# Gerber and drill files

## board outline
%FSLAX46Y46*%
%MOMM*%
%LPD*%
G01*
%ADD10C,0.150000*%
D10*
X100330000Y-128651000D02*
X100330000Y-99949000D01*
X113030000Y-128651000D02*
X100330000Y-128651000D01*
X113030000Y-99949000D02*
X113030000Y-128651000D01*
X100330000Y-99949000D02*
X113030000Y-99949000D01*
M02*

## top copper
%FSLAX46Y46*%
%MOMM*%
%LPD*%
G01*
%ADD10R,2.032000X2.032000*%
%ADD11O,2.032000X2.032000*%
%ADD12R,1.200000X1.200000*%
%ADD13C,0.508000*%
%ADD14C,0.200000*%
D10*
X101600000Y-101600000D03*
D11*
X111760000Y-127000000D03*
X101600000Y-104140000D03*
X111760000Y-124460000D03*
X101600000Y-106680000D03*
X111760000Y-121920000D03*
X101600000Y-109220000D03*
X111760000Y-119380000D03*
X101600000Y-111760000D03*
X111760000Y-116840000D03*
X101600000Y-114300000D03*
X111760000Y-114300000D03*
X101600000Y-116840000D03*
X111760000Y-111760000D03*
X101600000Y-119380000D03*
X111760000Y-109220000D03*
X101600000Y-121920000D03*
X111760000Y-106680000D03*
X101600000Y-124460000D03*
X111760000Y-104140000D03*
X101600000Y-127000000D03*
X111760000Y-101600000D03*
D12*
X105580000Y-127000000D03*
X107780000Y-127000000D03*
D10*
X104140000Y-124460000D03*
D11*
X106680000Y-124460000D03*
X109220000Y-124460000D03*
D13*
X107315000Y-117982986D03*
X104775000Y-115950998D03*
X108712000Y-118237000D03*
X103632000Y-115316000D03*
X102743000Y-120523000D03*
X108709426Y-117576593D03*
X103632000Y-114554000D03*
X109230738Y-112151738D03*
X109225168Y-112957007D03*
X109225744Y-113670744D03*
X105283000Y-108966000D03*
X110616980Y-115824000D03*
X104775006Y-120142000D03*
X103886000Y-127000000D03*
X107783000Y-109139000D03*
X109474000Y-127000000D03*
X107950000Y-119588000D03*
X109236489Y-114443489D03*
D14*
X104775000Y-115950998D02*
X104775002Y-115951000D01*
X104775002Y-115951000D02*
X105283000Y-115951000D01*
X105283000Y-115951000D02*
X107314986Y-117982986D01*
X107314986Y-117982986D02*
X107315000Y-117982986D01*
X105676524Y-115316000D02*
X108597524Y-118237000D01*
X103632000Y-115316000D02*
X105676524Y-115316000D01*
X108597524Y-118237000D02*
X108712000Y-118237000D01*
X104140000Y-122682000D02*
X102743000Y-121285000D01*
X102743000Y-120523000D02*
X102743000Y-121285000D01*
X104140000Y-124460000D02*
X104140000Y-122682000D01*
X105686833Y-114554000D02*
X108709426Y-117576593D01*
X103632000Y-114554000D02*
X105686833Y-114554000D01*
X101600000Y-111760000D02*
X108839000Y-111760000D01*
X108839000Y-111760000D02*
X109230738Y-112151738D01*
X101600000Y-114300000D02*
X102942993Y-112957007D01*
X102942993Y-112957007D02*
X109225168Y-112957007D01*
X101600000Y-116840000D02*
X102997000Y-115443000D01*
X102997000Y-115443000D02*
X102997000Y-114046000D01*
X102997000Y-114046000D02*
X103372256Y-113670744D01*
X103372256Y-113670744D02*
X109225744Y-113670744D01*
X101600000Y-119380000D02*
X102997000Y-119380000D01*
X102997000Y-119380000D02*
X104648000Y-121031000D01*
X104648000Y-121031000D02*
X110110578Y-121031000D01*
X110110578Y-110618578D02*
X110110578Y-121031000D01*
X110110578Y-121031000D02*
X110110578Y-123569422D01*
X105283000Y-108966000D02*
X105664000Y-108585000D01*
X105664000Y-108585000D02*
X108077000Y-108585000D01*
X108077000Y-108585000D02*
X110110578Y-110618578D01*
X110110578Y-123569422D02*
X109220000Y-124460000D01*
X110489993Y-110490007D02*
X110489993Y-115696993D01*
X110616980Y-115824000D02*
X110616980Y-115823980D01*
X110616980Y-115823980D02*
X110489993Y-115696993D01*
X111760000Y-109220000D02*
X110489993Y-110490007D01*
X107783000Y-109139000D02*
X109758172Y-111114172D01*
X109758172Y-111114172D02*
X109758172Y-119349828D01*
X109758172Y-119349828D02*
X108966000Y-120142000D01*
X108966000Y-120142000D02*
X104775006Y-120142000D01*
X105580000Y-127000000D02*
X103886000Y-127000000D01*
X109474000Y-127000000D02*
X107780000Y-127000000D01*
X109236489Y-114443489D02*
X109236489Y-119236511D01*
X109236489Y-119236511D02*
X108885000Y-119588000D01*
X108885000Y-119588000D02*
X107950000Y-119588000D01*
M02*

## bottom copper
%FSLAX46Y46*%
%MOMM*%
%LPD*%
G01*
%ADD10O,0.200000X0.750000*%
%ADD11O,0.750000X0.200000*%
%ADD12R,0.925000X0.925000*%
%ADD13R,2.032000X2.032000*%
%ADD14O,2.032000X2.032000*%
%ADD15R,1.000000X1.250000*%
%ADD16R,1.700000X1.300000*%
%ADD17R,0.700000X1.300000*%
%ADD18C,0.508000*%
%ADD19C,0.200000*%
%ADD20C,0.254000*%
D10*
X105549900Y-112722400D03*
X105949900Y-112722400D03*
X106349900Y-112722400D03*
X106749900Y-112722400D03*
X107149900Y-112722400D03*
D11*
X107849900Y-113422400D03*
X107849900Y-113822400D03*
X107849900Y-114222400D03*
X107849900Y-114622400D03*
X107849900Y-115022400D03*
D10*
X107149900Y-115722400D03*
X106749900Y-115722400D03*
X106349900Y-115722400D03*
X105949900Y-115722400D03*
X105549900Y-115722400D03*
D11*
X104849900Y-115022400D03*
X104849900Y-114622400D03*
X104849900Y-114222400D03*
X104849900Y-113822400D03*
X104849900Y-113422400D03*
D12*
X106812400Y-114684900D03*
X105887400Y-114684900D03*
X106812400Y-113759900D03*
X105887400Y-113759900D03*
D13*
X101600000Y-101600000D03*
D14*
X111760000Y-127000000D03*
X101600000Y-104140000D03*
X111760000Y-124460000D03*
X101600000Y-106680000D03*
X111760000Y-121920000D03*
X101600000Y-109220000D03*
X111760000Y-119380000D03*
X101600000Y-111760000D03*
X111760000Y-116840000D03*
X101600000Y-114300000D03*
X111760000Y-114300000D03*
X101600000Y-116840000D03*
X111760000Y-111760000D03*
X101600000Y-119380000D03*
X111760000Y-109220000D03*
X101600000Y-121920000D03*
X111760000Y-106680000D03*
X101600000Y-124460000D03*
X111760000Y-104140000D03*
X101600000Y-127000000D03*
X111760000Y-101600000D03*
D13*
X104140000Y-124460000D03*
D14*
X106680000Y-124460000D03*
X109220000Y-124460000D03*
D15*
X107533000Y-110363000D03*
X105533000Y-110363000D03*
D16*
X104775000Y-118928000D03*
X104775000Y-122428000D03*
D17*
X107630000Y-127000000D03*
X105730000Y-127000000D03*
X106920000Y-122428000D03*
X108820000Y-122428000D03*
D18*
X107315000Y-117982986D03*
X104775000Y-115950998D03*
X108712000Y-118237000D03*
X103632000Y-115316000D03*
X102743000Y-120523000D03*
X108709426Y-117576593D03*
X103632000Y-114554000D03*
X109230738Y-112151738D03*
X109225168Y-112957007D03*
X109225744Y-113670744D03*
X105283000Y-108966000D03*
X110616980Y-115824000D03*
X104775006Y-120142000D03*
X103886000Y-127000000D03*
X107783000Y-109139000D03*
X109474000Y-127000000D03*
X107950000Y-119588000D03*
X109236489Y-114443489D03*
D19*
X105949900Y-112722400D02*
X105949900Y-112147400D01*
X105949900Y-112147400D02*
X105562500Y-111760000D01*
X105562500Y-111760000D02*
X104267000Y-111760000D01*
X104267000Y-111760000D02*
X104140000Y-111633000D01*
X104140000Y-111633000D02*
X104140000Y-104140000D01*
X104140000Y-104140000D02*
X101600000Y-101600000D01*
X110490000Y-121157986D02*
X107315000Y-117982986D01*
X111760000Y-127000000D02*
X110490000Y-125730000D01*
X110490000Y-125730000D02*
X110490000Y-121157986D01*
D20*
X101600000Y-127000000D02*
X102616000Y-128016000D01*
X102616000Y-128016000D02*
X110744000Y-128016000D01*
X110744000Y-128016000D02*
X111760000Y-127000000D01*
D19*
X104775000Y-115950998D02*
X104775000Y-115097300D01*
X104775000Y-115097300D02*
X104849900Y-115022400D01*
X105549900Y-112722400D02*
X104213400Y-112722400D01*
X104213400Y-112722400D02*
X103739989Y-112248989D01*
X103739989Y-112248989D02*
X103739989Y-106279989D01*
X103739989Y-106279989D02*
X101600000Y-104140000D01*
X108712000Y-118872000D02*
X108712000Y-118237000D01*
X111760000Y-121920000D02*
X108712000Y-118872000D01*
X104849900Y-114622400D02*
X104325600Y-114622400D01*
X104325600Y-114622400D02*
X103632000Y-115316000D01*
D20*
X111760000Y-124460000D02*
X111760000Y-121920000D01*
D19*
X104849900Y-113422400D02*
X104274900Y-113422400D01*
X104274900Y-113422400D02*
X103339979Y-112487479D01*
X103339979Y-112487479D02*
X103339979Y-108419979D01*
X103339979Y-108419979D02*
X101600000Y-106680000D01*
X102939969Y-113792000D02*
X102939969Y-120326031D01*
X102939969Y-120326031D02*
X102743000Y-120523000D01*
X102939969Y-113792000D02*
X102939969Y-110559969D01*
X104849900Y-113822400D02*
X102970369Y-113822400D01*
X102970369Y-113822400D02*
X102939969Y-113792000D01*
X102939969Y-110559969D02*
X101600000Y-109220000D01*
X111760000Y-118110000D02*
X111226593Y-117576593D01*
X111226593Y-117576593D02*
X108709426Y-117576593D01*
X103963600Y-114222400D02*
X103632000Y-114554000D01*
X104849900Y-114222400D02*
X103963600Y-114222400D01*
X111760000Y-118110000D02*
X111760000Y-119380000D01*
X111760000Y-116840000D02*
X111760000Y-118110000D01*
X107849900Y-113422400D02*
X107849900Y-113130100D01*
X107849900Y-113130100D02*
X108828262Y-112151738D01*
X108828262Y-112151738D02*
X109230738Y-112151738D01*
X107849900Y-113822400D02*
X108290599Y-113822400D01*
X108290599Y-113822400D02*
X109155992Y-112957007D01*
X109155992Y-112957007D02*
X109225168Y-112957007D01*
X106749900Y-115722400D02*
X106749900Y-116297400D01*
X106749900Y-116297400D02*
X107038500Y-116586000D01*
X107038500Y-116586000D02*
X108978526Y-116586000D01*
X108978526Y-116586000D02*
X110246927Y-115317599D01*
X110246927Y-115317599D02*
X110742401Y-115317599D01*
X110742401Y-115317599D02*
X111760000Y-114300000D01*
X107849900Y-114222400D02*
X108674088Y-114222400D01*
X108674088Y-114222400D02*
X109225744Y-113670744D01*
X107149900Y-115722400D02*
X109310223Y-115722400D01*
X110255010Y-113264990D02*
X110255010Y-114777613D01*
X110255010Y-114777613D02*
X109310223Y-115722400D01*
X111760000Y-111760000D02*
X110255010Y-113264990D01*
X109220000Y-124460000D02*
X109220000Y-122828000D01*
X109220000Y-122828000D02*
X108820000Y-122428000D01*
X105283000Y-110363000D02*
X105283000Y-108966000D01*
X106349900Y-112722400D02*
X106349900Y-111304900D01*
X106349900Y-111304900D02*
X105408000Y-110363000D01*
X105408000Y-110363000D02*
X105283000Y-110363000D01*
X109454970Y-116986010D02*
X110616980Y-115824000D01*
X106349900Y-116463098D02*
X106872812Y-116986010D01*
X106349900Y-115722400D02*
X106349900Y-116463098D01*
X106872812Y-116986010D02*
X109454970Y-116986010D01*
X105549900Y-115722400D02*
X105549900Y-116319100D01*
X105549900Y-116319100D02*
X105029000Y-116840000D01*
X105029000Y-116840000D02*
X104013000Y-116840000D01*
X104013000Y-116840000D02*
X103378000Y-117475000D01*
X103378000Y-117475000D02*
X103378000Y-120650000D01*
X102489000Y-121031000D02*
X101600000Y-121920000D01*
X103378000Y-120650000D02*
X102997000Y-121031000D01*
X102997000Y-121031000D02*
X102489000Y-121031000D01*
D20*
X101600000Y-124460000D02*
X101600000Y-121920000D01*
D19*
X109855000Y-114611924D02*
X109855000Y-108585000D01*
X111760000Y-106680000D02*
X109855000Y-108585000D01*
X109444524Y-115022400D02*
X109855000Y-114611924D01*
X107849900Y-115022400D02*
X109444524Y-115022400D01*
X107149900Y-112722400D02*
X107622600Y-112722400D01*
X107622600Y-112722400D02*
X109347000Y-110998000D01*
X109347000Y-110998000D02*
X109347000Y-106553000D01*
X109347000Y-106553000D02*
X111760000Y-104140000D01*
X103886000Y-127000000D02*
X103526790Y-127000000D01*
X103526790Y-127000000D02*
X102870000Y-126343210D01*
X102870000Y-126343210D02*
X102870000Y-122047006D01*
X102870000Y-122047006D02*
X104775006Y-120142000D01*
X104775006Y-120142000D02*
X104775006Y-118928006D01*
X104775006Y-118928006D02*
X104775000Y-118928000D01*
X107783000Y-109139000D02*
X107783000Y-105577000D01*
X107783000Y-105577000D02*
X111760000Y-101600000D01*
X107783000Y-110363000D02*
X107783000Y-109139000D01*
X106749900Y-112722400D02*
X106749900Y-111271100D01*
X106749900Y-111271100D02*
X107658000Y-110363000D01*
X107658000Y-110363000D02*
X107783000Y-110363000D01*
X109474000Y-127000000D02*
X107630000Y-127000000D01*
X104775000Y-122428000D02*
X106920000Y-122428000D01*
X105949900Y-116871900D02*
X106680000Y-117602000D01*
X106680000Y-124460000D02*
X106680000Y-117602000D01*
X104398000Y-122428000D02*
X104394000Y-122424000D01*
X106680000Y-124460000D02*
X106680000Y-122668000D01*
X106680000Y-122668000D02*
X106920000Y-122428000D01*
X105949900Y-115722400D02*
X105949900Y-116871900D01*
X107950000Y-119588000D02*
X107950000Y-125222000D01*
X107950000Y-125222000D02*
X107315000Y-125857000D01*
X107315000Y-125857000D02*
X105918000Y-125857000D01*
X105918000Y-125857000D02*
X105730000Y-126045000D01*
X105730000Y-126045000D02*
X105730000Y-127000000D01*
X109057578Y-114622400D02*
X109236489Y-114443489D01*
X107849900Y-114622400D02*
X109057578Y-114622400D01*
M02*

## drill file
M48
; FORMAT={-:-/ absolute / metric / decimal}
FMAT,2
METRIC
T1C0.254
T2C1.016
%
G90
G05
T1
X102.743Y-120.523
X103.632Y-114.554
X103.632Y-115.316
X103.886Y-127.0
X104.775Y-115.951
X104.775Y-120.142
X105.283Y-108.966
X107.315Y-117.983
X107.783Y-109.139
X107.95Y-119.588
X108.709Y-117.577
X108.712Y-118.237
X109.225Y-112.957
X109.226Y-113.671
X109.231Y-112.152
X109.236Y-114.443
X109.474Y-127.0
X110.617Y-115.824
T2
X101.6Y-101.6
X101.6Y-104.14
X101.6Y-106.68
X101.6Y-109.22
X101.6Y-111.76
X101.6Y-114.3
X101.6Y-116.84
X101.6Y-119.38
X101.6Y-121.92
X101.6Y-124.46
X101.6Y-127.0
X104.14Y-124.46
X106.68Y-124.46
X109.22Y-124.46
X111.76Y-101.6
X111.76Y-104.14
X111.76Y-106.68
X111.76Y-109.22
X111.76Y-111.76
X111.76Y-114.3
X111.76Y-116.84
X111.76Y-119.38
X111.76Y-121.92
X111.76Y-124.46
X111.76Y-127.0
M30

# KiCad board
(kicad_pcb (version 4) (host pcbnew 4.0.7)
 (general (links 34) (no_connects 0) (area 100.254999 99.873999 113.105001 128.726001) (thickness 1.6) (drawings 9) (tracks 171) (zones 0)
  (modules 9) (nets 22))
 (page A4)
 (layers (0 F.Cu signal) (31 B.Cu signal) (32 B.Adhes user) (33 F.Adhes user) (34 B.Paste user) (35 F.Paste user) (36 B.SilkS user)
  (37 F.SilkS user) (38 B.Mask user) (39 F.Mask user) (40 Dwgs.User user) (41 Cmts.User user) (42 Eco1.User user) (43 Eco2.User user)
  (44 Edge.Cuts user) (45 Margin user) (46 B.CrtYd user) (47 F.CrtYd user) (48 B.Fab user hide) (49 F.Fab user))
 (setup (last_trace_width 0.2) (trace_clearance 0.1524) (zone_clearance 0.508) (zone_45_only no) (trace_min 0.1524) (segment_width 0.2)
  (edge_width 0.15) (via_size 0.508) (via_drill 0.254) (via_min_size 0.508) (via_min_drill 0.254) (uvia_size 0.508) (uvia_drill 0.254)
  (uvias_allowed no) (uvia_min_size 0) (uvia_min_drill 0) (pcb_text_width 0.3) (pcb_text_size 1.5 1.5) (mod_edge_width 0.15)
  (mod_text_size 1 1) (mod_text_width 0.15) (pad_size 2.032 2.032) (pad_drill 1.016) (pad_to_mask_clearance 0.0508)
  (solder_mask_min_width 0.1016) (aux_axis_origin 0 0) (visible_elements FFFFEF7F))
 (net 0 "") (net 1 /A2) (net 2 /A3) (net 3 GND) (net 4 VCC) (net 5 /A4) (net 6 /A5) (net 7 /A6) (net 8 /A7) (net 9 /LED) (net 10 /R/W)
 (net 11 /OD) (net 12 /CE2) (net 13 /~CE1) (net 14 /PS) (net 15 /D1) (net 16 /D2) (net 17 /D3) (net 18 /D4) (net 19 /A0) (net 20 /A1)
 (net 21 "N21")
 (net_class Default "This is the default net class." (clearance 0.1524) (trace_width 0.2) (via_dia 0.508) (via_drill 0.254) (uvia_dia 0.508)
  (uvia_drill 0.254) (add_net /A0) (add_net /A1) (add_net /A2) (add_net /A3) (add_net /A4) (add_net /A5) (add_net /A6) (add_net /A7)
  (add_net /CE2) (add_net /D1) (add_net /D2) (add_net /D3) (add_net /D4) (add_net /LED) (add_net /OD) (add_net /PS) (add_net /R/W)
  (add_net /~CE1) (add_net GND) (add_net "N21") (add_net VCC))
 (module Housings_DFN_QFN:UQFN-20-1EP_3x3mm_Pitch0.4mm (layer B.Cu) (at 106.3499 114.2224 270) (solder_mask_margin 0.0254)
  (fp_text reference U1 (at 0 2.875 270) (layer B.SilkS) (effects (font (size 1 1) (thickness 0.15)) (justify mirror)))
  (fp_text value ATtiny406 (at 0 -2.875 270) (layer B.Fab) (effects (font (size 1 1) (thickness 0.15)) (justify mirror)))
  (pad 1 smd oval (at -1.5 0.8 270) (size 0.75 0.2) (layers B.Cu B.Paste B.Mask) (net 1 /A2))
  (pad 2 smd oval (at -1.5 0.4 270) (size 0.75 0.2) (layers B.Cu B.Paste B.Mask) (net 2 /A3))
  (pad 3 smd oval (at -1.5 0 270) (size 0.75 0.2) (layers B.Cu B.Paste B.Mask) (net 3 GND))
  (pad 4 smd oval (at -1.5 -0.4 270) (size 0.75 0.2) (layers B.Cu B.Paste B.Mask) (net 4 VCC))
  (pad 5 smd oval (at -1.5 -0.8 270) (size 0.75 0.2) (layers B.Cu B.Paste B.Mask) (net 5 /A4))
  (pad 6 smd oval (at -0.8 -1.5 180) (size 0.75 0.2) (layers B.Cu B.Paste B.Mask) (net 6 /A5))
  (pad 7 smd oval (at -0.4 -1.5 180) (size 0.75 0.2) (layers B.Cu B.Paste B.Mask) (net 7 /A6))
  (pad 8 smd oval (at 0 -1.5 180) (size 0.75 0.2) (layers B.Cu B.Paste B.Mask) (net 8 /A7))
  (pad 9 smd oval (at 0.4 -1.5 180) (size 0.75 0.2) (layers B.Cu B.Paste B.Mask) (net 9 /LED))
  (pad 10 smd oval (at 0.8 -1.5 180) (size 0.75 0.2) (layers B.Cu B.Paste B.Mask) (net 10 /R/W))
  (pad 11 smd oval (at 1.5 -0.8 270) (size 0.75 0.2) (layers B.Cu B.Paste B.Mask) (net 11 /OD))
  (pad 12 smd oval (at 1.5 -0.4 270) (size 0.75 0.2) (layers B.Cu B.Paste B.Mask) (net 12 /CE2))
  (pad 13 smd oval (at 1.5 0 270) (size 0.75 0.2) (layers B.Cu B.Paste B.Mask) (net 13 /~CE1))
  (pad 14 smd oval (at 1.5 0.4 270) (size 0.75 0.2) (layers B.Cu B.Paste B.Mask) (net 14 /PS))
  (pad 15 smd oval (at 1.5 0.8 270) (size 0.75 0.2) (layers B.Cu B.Paste B.Mask) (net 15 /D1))
  (pad 16 smd oval (at 0.8 1.5 180) (size 0.75 0.2) (layers B.Cu B.Paste B.Mask) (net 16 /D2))
  (pad 17 smd oval (at 0.4 1.5 180) (size 0.75 0.2) (layers B.Cu B.Paste B.Mask) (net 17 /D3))
  (pad 18 smd oval (at 0 1.5 180) (size 0.75 0.2) (layers B.Cu B.Paste B.Mask) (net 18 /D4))
  (pad 19 smd oval (at -0.4 1.5 180) (size 0.75 0.2) (layers B.Cu B.Paste B.Mask) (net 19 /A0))
  (pad 20 smd oval (at -0.8 1.5 180) (size 0.75 0.2) (layers B.Cu B.Paste B.Mask) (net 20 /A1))
  (pad 21 smd rect (at 0.4625 -0.4625 270) (size 0.925 0.925) (layers B.Cu B.Paste B.Mask) (solder_paste_margin_ratio -0.2))
  (pad 21 smd rect (at 0.4625 0.4625 270) (size 0.925 0.925) (layers B.Cu B.Paste B.Mask) (solder_paste_margin_ratio -0.2))
  (pad 21 smd rect (at -0.4625 -0.4625 270) (size 0.925 0.925) (layers B.Cu B.Paste B.Mask) (solder_paste_margin_ratio -0.2))
  (pad 21 smd rect (at -0.4625 0.4625 270) (size 0.925 0.925) (layers B.Cu B.Paste B.Mask) (solder_paste_margin_ratio -0.2)))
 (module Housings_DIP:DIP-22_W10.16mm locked (layer F.Cu) (at 101.6 101.6)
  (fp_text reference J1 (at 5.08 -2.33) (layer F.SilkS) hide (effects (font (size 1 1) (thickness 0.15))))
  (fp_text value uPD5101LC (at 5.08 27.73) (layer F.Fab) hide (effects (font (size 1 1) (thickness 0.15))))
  (pad 1 thru_hole rect (at 0 0) (size 2.032 2.032) (drill 1.016) (layers *.Cu *.Mask) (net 2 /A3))
  (pad 12 thru_hole oval (at 10.16 25.4) (size 2.032 2.032) (drill 1.016) (layers *.Cu *.Mask) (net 16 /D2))
  (pad 2 thru_hole oval (at 0 2.54) (size 2.032 2.032) (drill 1.016) (layers *.Cu *.Mask) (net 1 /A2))
  (pad 13 thru_hole oval (at 10.16 22.86) (size 2.032 2.032) (drill 1.016) (layers *.Cu *.Mask) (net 17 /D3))
  (pad 3 thru_hole oval (at 0 5.08) (size 2.032 2.032) (drill 1.016) (layers *.Cu *.Mask) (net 20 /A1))
  (pad 14 thru_hole oval (at 10.16 20.32) (size 2.032 2.032) (drill 1.016) (layers *.Cu *.Mask) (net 17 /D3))
  (pad 4 thru_hole oval (at 0 7.62) (size 2.032 2.032) (drill 1.016) (layers *.Cu *.Mask) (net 19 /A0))
  (pad 15 thru_hole oval (at 10.16 17.78) (size 2.032 2.032) (drill 1.016) (layers *.Cu *.Mask) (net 18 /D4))
  (pad 5 thru_hole oval (at 0 10.16) (size 2.032 2.032) (drill 1.016) (layers *.Cu *.Mask) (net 6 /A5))
  (pad 16 thru_hole oval (at 10.16 15.24) (size 2.032 2.032) (drill 1.016) (layers *.Cu *.Mask) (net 18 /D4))
  (pad 6 thru_hole oval (at 0 12.7) (size 2.032 2.032) (drill 1.016) (layers *.Cu *.Mask) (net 7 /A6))
  (pad 17 thru_hole oval (at 10.16 12.7) (size 2.032 2.032) (drill 1.016) (layers *.Cu *.Mask) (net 12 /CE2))
  (pad 7 thru_hole oval (at 0 15.24) (size 2.032 2.032) (drill 1.016) (layers *.Cu *.Mask) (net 8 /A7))
  (pad 18 thru_hole oval (at 10.16 10.16) (size 2.032 2.032) (drill 1.016) (layers *.Cu *.Mask) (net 11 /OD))
  (pad 8 thru_hole oval (at 0 17.78) (size 2.032 2.032) (drill 1.016) (layers *.Cu *.Mask) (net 3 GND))
  (pad 19 thru_hole oval (at 10.16 7.62) (size 2.032 2.032) (drill 1.016) (layers *.Cu *.Mask) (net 13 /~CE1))
  (pad 9 thru_hole oval (at 0 20.32) (size 2.032 2.032) (drill 1.016) (layers *.Cu *.Mask) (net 15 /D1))
  (pad 20 thru_hole oval (at 10.16 5.08) (size 2.032 2.032) (drill 1.016) (layers *.Cu *.Mask) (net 10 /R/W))
  (pad 10 thru_hole oval (at 0 22.86) (size 2.032 2.032) (drill 1.016) (layers *.Cu *.Mask) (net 15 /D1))
  (pad 21 thru_hole oval (at 10.16 2.54) (size 2.032 2.032) (drill 1.016) (layers *.Cu *.Mask) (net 5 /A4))
  (pad 11 thru_hole oval (at 0 25.4) (size 2.032 2.032) (drill 1.016) (layers *.Cu *.Mask) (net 16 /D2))
  (pad 22 thru_hole oval (at 10.16 0) (size 2.032 2.032) (drill 1.016) (layers *.Cu *.Mask) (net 4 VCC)))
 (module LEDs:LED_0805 (layer F.Cu) (at 106.68 127 180)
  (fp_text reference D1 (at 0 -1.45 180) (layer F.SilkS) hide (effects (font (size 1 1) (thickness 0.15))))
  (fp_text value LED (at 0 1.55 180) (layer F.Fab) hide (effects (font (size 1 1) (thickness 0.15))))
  (pad 2 smd rect (at 1.1 0) (size 1.2 1.2) (layers F.Cu F.Paste F.Mask) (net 4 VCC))
  (pad 1 smd rect (at -1.1 0) (size 1.2 1.2) (layers F.Cu F.Paste F.Mask) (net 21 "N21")))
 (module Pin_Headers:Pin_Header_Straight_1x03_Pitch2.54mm (layer F.Cu) (at 104.14 124.46 90)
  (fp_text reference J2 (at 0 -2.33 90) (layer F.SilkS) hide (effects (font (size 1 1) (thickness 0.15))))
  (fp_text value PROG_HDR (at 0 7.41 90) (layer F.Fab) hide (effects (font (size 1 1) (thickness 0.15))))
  (pad 1 thru_hole rect (at 0 0 90) (size 2.032 2.032) (drill 1.016) (layers *.Cu *.Mask) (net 19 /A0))
  (pad 2 thru_hole oval (at 0 2.54 90) (size 2.032 2.032) (drill 1.016) (layers *.Cu *.Mask) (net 14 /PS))
  (pad 3 thru_hole oval (at 0 5.08 90) (size 2.032 2.032) (drill 1.016) (layers *.Cu *.Mask) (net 3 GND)))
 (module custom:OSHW (layer F.Cu) (at 107.95 103.632 270)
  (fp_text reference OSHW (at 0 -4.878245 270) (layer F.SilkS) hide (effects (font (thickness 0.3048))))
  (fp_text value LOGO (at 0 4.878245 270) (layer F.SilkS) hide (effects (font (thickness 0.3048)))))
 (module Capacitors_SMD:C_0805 (layer B.Cu) (at 106.533 110.363 180)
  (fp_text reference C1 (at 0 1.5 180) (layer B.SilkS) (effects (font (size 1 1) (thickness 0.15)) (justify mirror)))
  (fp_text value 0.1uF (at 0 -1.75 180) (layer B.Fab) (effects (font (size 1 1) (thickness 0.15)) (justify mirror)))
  (pad 1 smd rect (at -1 0 180) (size 1 1.25) (layers B.Cu B.Paste B.Mask) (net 4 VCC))
  (pad 2 smd rect (at 1 0 180) (size 1 1.25) (layers B.Cu B.Paste B.Mask) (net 3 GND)))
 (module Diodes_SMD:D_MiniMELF (layer B.Cu) (at 104.775 120.678 270)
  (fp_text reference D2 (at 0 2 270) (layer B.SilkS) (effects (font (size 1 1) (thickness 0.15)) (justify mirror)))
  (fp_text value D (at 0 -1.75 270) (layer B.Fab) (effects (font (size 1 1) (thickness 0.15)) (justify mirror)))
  (pad 1 smd rect (at -1.75 0 270) (size 1.3 1.7) (layers B.Cu B.Paste B.Mask) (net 4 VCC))
  (pad 2 smd rect (at 1.75 0 270) (size 1.3 1.7) (layers B.Cu B.Paste B.Mask) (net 14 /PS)))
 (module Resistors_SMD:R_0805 (layer B.Cu) (at 106.68 127 180)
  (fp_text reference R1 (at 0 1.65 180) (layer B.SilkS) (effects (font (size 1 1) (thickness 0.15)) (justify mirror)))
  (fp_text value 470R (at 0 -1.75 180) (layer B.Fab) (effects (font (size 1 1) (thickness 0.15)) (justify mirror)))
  (pad 1 smd rect (at -0.95 0 180) (size 0.7 1.3) (layers B.Cu B.Paste B.Mask) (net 21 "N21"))
  (pad 2 smd rect (at 0.95 0 180) (size 0.7 1.3) (layers B.Cu B.Paste B.Mask) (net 9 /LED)))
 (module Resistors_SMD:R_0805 (layer B.Cu) (at 107.87 122.428)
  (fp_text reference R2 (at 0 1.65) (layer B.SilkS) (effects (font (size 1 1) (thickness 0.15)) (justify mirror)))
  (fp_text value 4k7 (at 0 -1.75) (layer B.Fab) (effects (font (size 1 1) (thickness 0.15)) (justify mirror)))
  (pad 1 smd rect (at -0.95 0) (size 0.7 1.3) (layers B.Cu B.Paste B.Mask) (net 14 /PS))
  (pad 2 smd rect (at 0.95 0) (size 0.7 1.3) (layers B.Cu B.Paste B.Mask) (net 3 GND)))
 (gr_line (start 100.33 128.651) (end 100.33 99.949) (layer Edge.Cuts) (width 0.15))
 (gr_line (start 113.03 128.651) (end 100.33 128.651) (layer Edge.Cuts) (width 0.15))
 (gr_line (start 113.03 99.949) (end 113.03 128.651) (layer Edge.Cuts) (width 0.15))
 (gr_line (start 100.33 99.949) (end 113.03 99.949) (layer Edge.Cuts) (width 0.15))
 (segment (start 105.9499 112.7224) (end 105.9499 112.1474) (width 0.2) (layer B.Cu) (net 2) (status 10))
 (segment (start 105.9499 112.1474) (end 105.5625 111.76) (width 0.2) (layer B.Cu) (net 2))
 (segment (start 105.5625 111.76) (end 104.267 111.76) (width 0.2) (layer B.Cu) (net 2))
 (segment (start 104.267 111.76) (end 104.14 111.633) (width 0.2) (layer B.Cu) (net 2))
 (segment (start 104.14 111.633) (end 104.14 104.14) (width 0.2) (layer B.Cu) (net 2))
 (segment (start 104.14 104.14) (end 101.6 101.6) (width 0.2) (layer B.Cu) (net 2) (status 20))
 (segment (start 104.775 115.950998) (end 104.775002 115.951) (width 0.2) (layer F.Cu) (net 16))
 (segment (start 104.775002 115.951) (end 105.283 115.951) (width 0.2) (layer F.Cu) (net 16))
 (segment (start 105.283 115.951) (end 107.314986 117.982986) (width 0.2) (layer F.Cu) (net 16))
 (segment (start 107.314986 117.982986) (end 107.315 117.982986) (width 0.2) (layer F.Cu) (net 16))
 (segment (start 110.49 121.157986) (end 107.315 117.982986) (width 0.2) (layer B.Cu) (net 16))
 (segment (start 111.76 127) (end 110.49 125.73) (width 0.2) (layer B.Cu) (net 16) (status 10))
 (segment (start 110.49 125.73) (end 110.49 121.157986) (width 0.2) (layer B.Cu) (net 16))
 (via (at 107.315 117.982986) (size 0.508) (drill 0.254) (layers F.Cu B.Cu) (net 16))
 (segment (start 101.6 127) (end 102.616 128.016) (width 0.254) (layer B.Cu) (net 16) (status 10))
 (segment (start 102.616 128.016) (end 110.744 128.016) (width 0.254) (layer B.Cu) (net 16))
 (segment (start 110.744 128.016) (end 111.76 127) (width 0.254) (layer B.Cu) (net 16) (status 20))
 (segment (start 104.775 115.950998) (end 104.775 115.0973) (width 0.2) (layer B.Cu) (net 16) (status 20))
 (segment (start 104.775 115.0973) (end 104.8499 115.0224) (width 0.2) (layer B.Cu) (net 16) (status 30))
 (via (at 104.775 115.950998) (size 0.508) (drill 0.254) (layers F.Cu B.Cu) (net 16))
 (segment (start 105.5499 112.7224) (end 104.2134 112.7224) (width 0.2) (layer B.Cu) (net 1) (status 10))
 (segment (start 104.2134 112.7224) (end 103.739989 112.248989) (width 0.2) (layer B.Cu) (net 1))
 (segment (start 103.739989 112.248989) (end 103.739989 106.279989) (width 0.2) (layer B.Cu) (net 1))
 (segment (start 103.739989 106.279989) (end 101.6 104.14) (width 0.2) (layer B.Cu) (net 1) (status 20))
 (segment (start 105.676524 115.316) (end 108.597524 118.237) (width 0.2) (layer F.Cu) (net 17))
 (segment (start 103.632 115.316) (end 105.676524 115.316) (width 0.2) (layer F.Cu) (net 17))
 (segment (start 108.712 118.872) (end 108.712 118.237) (width 0.2) (layer B.Cu) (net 17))
 (via (at 108.712 118.237) (size 0.508) (drill 0.254) (layers F.Cu B.Cu) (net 17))
 (segment (start 108.597524 118.237) (end 108.712 118.237) (width 0.2) (layer F.Cu) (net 17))
 (segment (start 111.76 121.92) (end 108.712 118.872) (width 0.2) (layer B.Cu) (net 17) (status 10))
 (segment (start 104.8499 114.6224) (end 104.3256 114.6224) (width 0.2) (layer B.Cu) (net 17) (status 10))
 (segment (start 104.3256 114.6224) (end 103.632 115.316) (width 0.2) (layer B.Cu) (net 17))
 (via (at 103.632 115.316) (size 0.508) (drill 0.254) (layers F.Cu B.Cu) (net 17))
 (segment (start 111.76 124.46) (end 111.76 121.92) (width 0.254) (layer B.Cu) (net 17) (status 30))
 (segment (start 104.8499 113.4224) (end 104.2749 113.4224) (width 0.2) (layer B.Cu) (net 20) (status 10))
 (segment (start 104.2749 113.4224) (end 103.339979 112.487479) (width 0.2) (layer B.Cu) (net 20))
 (segment (start 103.339979 112.487479) (end 103.339979 108.419979) (width 0.2) (layer B.Cu) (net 20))
 (segment (start 103.339979 108.419979) (end 101.6 106.68) (width 0.2) (layer B.Cu) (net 20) (status 20))
 (segment (start 104.14 122.682) (end 102.743 121.285) (width 0.2) (layer F.Cu) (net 19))
 (segment (start 102.743 120.523) (end 102.743 121.285) (width 0.2) (layer F.Cu) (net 19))
 (segment (start 102.939969 113.792) (end 102.939969 120.326031) (width 0.2) (layer B.Cu) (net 19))
 (segment (start 102.939969 120.326031) (end 102.743 120.523) (width 0.2) (layer B.Cu) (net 19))
 (via (at 102.743 120.523) (size 0.508) (drill 0.254) (layers F.Cu B.Cu) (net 19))
 (segment (start 102.939969 113.792) (end 102.939969 110.559969) (width 0.2) (layer B.Cu) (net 19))
 (segment (start 104.8499 113.8224) (end 102.970369 113.8224) (width 0.2) (layer B.Cu) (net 19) (status 10))
 (segment (start 102.970369 113.8224) (end 102.939969 113.792) (width 0.2) (layer B.Cu) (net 19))
 (segment (start 104.14 124.46) (end 104.14 122.682) (width 0.2) (layer F.Cu) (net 19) (status 10))
 (segment (start 102.939969 110.559969) (end 101.6 109.22) (width 0.2) (layer B.Cu) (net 19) (status 20))
 (via (at 108.709426 117.576593) (size 0.508) (drill 0.254) (layers F.Cu B.Cu) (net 18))
 (segment (start 111.76 118.11) (end 111.226593 117.576593) (width 0.2) (layer B.Cu) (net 18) (status 20))
 (segment (start 105.686833 114.554) (end 108.709426 117.576593) (width 0.2) (layer F.Cu) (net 18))
 (segment (start 111.226593 117.576593) (end 108.709426 117.576593) (width 0.2) (layer B.Cu) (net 18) (status 10))
 (segment (start 103.632 114.554) (end 105.686833 114.554) (width 0.2) (layer F.Cu) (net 18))
 (segment (start 103.9636 114.2224) (end 103.632 114.554) (width 0.2) (layer B.Cu) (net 18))
 (segment (start 104.8499 114.2224) (end 103.9636 114.2224) (width 0.2) (layer B.Cu) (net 18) (status 10))
 (via (at 103.632 114.554) (size 0.508) (drill 0.254) (layers F.Cu B.Cu) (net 18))
 (segment (start 111.76 118.11) (end 111.76 119.38) (width 0.2) (layer B.Cu) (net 18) (status 20))
 (segment (start 111.76 116.84) (end 111.76 118.11) (width 0.2) (layer B.Cu) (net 18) (status 10))
 (segment (start 101.6 111.76) (end 108.839 111.76) (width 0.2) (layer F.Cu) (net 6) (status 10))
 (segment (start 108.839 111.76) (end 109.230738 112.151738) (width 0.2) (layer F.Cu) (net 6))
 (segment (start 107.8499 113.4224) (end 107.8499 113.1301) (width 0.2) (layer B.Cu) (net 6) (status 10))
 (segment (start 107.8499 113.1301) (end 108.828262 112.151738) (width 0.2) (layer B.Cu) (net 6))
 (segment (start 108.828262 112.151738) (end 109.230738 112.151738) (width 0.2) (layer B.Cu) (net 6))
 (via (at 109.230738 112.151738) (size 0.508) (drill 0.254) (layers F.Cu B.Cu) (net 6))
 (segment (start 101.6 114.3) (end 102.942993 112.957007) (width 0.2) (layer F.Cu) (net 7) (status 10))
 (segment (start 102.942993 112.957007) (end 109.225168 112.957007) (width 0.2) (layer F.Cu) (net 7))
 (segment (start 107.8499 113.8224) (end 108.290599 113.8224) (width 0.2) (layer B.Cu) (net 7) (status 10))
 (segment (start 108.290599 113.8224) (end 109.155992 112.957007) (width 0.2) (layer B.Cu) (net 7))
 (segment (start 109.155992 112.957007) (end 109.225168 112.957007) (width 0.2) (layer B.Cu) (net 7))
 (via (at 109.225168 112.957007) (size 0.508) (drill 0.254) (layers F.Cu B.Cu) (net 7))
 (segment (start 106.7499 115.7224) (end 106.7499 116.2974) (width 0.2) (layer B.Cu) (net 12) (status 10))
 (segment (start 106.7499 116.2974) (end 107.0385 116.586) (width 0.2) (layer B.Cu) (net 12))
 (segment (start 107.0385 116.586) (end 108.978526 116.586) (width 0.2) (layer B.Cu) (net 12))
 (segment (start 108.978526 116.586) (end 110.246927 115.317599) (width 0.2) (layer B.Cu) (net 12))
 (segment (start 110.246927 115.317599) (end 110.742401 115.317599) (width 0.2) (layer B.Cu) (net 12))
 (segment (start 110.742401 115.317599) (end 111.76 114.3) (width 0.2) (layer B.Cu) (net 12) (status 20))
 (segment (start 101.6 116.84) (end 102.997 115.443) (width 0.2) (layer F.Cu) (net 8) (status 10))
 (segment (start 102.997 115.443) (end 102.997 114.046) (width 0.2) (layer F.Cu) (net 8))
 (segment (start 102.997 114.046) (end 103.372256 113.670744) (width 0.2) (layer F.Cu) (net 8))
 (segment (start 103.372256 113.670744) (end 109.225744 113.670744) (width 0.2) (layer F.Cu) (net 8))
 (segment (start 107.8499 114.2224) (end 108.674088 114.2224) (width 0.2) (layer B.Cu) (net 8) (status 10))
 (segment (start 108.674088 114.2224) (end 109.225744 113.670744) (width 0.2) (layer B.Cu) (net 8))
 (via (at 109.225744 113.670744) (size 0.508) (drill 0.254) (layers F.Cu B.Cu) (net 8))
 (segment (start 107.1499 115.7224) (end 109.310223 115.7224) (width 0.2) (layer B.Cu) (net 11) (status 10))
 (segment (start 110.25501 113.26499) (end 110.25501 114.777613) (width 0.2) (layer B.Cu) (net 11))
 (segment (start 110.25501 114.777613) (end 109.310223 115.7224) (width 0.2) (layer B.Cu) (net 11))
 (segment (start 111.76 111.76) (end 110.25501 113.26499) (width 0.2) (layer B.Cu) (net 11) (status 10))
 (segment (start 101.6 119.38) (end 102.997 119.38) (width 0.2) (layer F.Cu) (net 3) (status 10))
 (segment (start 102.997 119.38) (end 104.648 121.031) (width 0.2) (layer F.Cu) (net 3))
 (segment (start 104.648 121.031) (end 110.110578 121.031) (width 0.2) (layer F.Cu) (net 3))
 (segment (start 110.110578 110.618578) (end 110.110578 121.031) (width 0.2) (layer F.Cu) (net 3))
 (segment (start 110.110578 121.031) (end 110.110578 123.569422) (width 0.2) (layer F.Cu) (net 3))
 (segment (start 105.283 108.966) (end 105.664 108.585) (width 0.2) (layer F.Cu) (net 3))
 (segment (start 105.664 108.585) (end 108.077 108.585) (width 0.2) (layer F.Cu) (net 3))
 (segment (start 108.077 108.585) (end 110.110578 110.618578) (width 0.2) (layer F.Cu) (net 3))
 (segment (start 110.110578 123.569422) (end 109.22 124.46) (width 0.2) (layer F.Cu) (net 3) (status 20))
 (segment (start 109.22 124.46) (end 109.22 122.828) (width 0.2) (layer B.Cu) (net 3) (status 10))
 (segment (start 109.22 122.828) (end 108.82 122.428) (width 0.2) (layer B.Cu) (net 3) (status 20))
 (via (at 105.283 108.966) (size 0.508) (drill 0.254) (layers F.Cu B.Cu) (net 3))
 (segment (start 105.283 110.363) (end 105.283 108.966) (width 0.2) (layer B.Cu) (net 3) (status 10))
 (segment (start 106.3499 112.7224) (end 106.3499 111.3049) (width 0.2) (layer B.Cu) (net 3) (status 10))
 (segment (start 106.3499 111.3049) (end 105.408 110.363) (width 0.2) (layer B.Cu) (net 3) (status 20))
 (segment (start 105.408 110.363) (end 105.283 110.363) (width 0.2) (layer B.Cu) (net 3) (status 30))
 (segment (start 110.489993 110.490007) (end 110.489993 115.696993) (width 0.2) (layer F.Cu) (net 13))
 (segment (start 110.61698 115.824) (end 110.61698 115.82398) (width 0.2) (layer F.Cu) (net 13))
 (segment (start 110.61698 115.82398) (end 110.489993 115.696993) (width 0.2) (layer F.Cu) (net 13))
 (segment (start 111.76 109.22) (end 110.489993 110.490007) (width 0.2) (layer F.Cu) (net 13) (status 10))
 (segment (start 109.45497 116.98601) (end 110.61698 115.824) (width 0.2) (layer B.Cu) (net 13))
 (segment (start 106.3499 116.463098) (end 106.872812 116.98601) (width 0.2) (layer B.Cu) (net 13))
 (segment (start 106.3499 115.7224) (end 106.3499 116.463098) (width 0.2) (layer B.Cu) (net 13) (status 10))
 (via (at 110.61698 115.824) (size 0.508) (drill 0.254) (layers F.Cu B.Cu) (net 13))
 (segment (start 106.872812 116.98601) (end 109.45497 116.98601) (width 0.2) (layer B.Cu) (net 13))
 (segment (start 105.5499 115.7224) (end 105.5499 116.3191) (width 0.2) (layer B.Cu) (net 15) (status 10))
 (segment (start 105.5499 116.3191) (end 105.029 116.84) (width 0.2) (layer B.Cu) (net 15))
 (segment (start 105.029 116.84) (end 104.013 116.84) (width 0.2) (layer B.Cu) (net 15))
 (segment (start 104.013 116.84) (end 103.378 117.475) (width 0.2) (layer B.Cu) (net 15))
 (segment (start 103.378 117.475) (end 103.378 120.65) (width 0.2) (layer B.Cu) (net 15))
 (segment (start 102.489 121.031) (end 101.6 121.92) (width 0.2) (layer B.Cu) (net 15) (status 20))
 (segment (start 103.378 120.65) (end 102.997 121.031) (width 0.2) (layer B.Cu) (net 15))
 (segment (start 102.997 121.031) (end 102.489 121.031) (width 0.2) (layer B.Cu) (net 15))
 (segment (start 101.6 124.46) (end 101.6 121.92) (width 0.254) (layer B.Cu) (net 15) (status 30))
 (segment (start 109.855 114.611924) (end 109.855 108.585) (width 0.2) (layer B.Cu) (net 10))
 (segment (start 111.76 106.68) (end 109.855 108.585) (width 0.2) (layer B.Cu) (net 10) (status 10))
 (segment (start 109.444524 115.0224) (end 109.855 114.611924) (width 0.2) (layer B.Cu) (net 10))
 (segment (start 107.8499 115.0224) (end 109.444524 115.0224) (width 0.2) (layer B.Cu) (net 10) (status 10))
 (segment (start 107.1499 112.7224) (end 107.6226 112.7224) (width 0.2) (layer B.Cu) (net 5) (status 10))
 (segment (start 107.6226 112.7224) (end 109.347 110.998) (width 0.2) (layer B.Cu) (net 5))
 (segment (start 109.347 110.998) (end 109.347 106.553) (width 0.2) (layer B.Cu) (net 5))
 (segment (start 109.347 106.553) (end 111.76 104.14) (width 0.2) (layer B.Cu) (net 5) (status 20))
 (segment (start 107.783 109.139) (end 109.758172 111.114172) (width 0.2) (layer F.Cu) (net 4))
 (segment (start 109.758172 111.114172) (end 109.758172 119.349828) (width 0.2) (layer F.Cu) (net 4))
 (segment (start 109.758172 119.349828) (end 108.966 120.142) (width 0.2) (layer F.Cu) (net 4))
 (segment (start 108.966 120.142) (end 104.775006 120.142) (width 0.2) (layer F.Cu) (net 4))
 (segment (start 103.886 127) (end 103.52679 127) (width 0.2) (layer B.Cu) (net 4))
 (segment (start 103.52679 127) (end 102.87 126.34321) (width 0.2) (layer B.Cu) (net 4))
 (segment (start 102.87 126.34321) (end 102.87 122.047006) (width 0.2) (layer B.Cu) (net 4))
 (segment (start 102.87 122.047006) (end 104.775006 120.142) (width 0.2) (layer B.Cu) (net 4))
 (segment (start 104.775006 120.142) (end 104.775006 118.928006) (width 0.2) (layer B.Cu) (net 4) (status 20))
 (segment (start 104.775006 118.928006) (end 104.775 118.928) (width 0.2) (layer B.Cu) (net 4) (status 30))
 (via (at 104.775006 120.142) (size 0.508) (drill 0.254) (layers F.Cu B.Cu) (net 4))
 (segment (start 105.58 127) (end 103.886 127) (width 0.2) (layer F.Cu) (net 4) (status 10))
 (via (at 103.886 127) (size 0.508) (drill 0.254) (layers F.Cu B.Cu) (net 4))
 (segment (start 107.783 109.139) (end 107.783 105.577) (width 0.2) (layer B.Cu) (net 4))
 (segment (start 107.783 105.577) (end 111.76 101.6) (width 0.2) (layer B.Cu) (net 4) (status 20))
 (via (at 107.783 109.139) (size 0.508) (drill 0.254) (layers F.Cu B.Cu) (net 4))
 (segment (start 107.783 110.363) (end 107.783 109.139) (width 0.2) (layer B.Cu) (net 4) (status 10))
 (segment (start 106.7499 112.7224) (end 106.7499 111.2711) (width 0.2) (layer B.Cu) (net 4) (status 10))
 (segment (start 106.7499 111.2711) (end 107.658 110.363) (width 0.2) (layer B.Cu) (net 4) (status 20))
 (segment (start 107.658 110.363) (end 107.783 110.363) (width 0.2) (layer B.Cu) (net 4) (status 30))
 (segment (start 109.474 127) (end 107.78 127) (width 0.2) (layer F.Cu) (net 21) (status 20))
 (segment (start 109.474 127) (end 107.63 127) (width 0.2) (layer B.Cu) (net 21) (status 20))
 (via (at 109.474 127) (size 0.508) (drill 0.254) (layers F.Cu B.Cu) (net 21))
 (segment (start 104.775 122.428) (end 106.92 122.428) (width 0.2) (layer B.Cu) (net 14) (status 30))
 (segment (start 105.9499 116.8719) (end 106.68 117.602) (width 0.2) (layer B.Cu) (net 14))
 (segment (start 106.68 124.46) (end 106.68 117.602) (width 0.2) (layer B.Cu) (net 14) (status 10))
 (segment (start 104.398 122.428) (end 104.394 122.424) (width 0.2) (layer B.Cu) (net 14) (status 30))
 (segment (start 106.68 124.46) (end 106.68 122.668) (width 0.2) (layer B.Cu) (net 14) (status 30))
 (segment (start 106.68 122.668) (end 106.92 122.428) (width 0.2) (layer B.Cu) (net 14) (status 30))
 (segment (start 105.9499 115.7224) (end 105.9499 116.8719) (width 0.2) (layer B.Cu) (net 14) (status 10))
 (segment (start 107.95 119.588) (end 107.95 125.222) (width 0.2) (layer B.Cu) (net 9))
 (segment (start 107.95 125.222) (end 107.315 125.857) (width 0.2) (layer B.Cu) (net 9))
 (segment (start 107.315 125.857) (end 105.918 125.857) (width 0.2) (layer B.Cu) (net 9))
 (segment (start 105.918 125.857) (end 105.73 126.045) (width 0.2) (layer B.Cu) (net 9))
 (segment (start 105.73 126.045) (end 105.73 127) (width 0.2) (layer B.Cu) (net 9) (status 20))
 (segment (start 109.236489 114.443489) (end 109.236489 119.236511) (width 0.2) (layer F.Cu) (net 9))
 (segment (start 109.236489 119.236511) (end 108.885 119.588) (width 0.2) (layer F.Cu) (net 9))
 (segment (start 108.885 119.588) (end 107.95 119.588) (width 0.2) (layer F.Cu) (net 9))
 (via (at 107.95 119.588) (size 0.508) (drill 0.254) (layers F.Cu B.Cu) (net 9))
 (via (at 109.236489 114.443489) (size 0.508) (drill 0.254) (layers F.Cu B.Cu) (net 9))
 (segment (start 109.057578 114.6224) (end 109.236489 114.443489) (width 0.2) (layer B.Cu) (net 9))
 (segment (start 107.8499 114.6224) (end 109.057578 114.6224) (width 0.2) (layer B.Cu) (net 9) (status 10)))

